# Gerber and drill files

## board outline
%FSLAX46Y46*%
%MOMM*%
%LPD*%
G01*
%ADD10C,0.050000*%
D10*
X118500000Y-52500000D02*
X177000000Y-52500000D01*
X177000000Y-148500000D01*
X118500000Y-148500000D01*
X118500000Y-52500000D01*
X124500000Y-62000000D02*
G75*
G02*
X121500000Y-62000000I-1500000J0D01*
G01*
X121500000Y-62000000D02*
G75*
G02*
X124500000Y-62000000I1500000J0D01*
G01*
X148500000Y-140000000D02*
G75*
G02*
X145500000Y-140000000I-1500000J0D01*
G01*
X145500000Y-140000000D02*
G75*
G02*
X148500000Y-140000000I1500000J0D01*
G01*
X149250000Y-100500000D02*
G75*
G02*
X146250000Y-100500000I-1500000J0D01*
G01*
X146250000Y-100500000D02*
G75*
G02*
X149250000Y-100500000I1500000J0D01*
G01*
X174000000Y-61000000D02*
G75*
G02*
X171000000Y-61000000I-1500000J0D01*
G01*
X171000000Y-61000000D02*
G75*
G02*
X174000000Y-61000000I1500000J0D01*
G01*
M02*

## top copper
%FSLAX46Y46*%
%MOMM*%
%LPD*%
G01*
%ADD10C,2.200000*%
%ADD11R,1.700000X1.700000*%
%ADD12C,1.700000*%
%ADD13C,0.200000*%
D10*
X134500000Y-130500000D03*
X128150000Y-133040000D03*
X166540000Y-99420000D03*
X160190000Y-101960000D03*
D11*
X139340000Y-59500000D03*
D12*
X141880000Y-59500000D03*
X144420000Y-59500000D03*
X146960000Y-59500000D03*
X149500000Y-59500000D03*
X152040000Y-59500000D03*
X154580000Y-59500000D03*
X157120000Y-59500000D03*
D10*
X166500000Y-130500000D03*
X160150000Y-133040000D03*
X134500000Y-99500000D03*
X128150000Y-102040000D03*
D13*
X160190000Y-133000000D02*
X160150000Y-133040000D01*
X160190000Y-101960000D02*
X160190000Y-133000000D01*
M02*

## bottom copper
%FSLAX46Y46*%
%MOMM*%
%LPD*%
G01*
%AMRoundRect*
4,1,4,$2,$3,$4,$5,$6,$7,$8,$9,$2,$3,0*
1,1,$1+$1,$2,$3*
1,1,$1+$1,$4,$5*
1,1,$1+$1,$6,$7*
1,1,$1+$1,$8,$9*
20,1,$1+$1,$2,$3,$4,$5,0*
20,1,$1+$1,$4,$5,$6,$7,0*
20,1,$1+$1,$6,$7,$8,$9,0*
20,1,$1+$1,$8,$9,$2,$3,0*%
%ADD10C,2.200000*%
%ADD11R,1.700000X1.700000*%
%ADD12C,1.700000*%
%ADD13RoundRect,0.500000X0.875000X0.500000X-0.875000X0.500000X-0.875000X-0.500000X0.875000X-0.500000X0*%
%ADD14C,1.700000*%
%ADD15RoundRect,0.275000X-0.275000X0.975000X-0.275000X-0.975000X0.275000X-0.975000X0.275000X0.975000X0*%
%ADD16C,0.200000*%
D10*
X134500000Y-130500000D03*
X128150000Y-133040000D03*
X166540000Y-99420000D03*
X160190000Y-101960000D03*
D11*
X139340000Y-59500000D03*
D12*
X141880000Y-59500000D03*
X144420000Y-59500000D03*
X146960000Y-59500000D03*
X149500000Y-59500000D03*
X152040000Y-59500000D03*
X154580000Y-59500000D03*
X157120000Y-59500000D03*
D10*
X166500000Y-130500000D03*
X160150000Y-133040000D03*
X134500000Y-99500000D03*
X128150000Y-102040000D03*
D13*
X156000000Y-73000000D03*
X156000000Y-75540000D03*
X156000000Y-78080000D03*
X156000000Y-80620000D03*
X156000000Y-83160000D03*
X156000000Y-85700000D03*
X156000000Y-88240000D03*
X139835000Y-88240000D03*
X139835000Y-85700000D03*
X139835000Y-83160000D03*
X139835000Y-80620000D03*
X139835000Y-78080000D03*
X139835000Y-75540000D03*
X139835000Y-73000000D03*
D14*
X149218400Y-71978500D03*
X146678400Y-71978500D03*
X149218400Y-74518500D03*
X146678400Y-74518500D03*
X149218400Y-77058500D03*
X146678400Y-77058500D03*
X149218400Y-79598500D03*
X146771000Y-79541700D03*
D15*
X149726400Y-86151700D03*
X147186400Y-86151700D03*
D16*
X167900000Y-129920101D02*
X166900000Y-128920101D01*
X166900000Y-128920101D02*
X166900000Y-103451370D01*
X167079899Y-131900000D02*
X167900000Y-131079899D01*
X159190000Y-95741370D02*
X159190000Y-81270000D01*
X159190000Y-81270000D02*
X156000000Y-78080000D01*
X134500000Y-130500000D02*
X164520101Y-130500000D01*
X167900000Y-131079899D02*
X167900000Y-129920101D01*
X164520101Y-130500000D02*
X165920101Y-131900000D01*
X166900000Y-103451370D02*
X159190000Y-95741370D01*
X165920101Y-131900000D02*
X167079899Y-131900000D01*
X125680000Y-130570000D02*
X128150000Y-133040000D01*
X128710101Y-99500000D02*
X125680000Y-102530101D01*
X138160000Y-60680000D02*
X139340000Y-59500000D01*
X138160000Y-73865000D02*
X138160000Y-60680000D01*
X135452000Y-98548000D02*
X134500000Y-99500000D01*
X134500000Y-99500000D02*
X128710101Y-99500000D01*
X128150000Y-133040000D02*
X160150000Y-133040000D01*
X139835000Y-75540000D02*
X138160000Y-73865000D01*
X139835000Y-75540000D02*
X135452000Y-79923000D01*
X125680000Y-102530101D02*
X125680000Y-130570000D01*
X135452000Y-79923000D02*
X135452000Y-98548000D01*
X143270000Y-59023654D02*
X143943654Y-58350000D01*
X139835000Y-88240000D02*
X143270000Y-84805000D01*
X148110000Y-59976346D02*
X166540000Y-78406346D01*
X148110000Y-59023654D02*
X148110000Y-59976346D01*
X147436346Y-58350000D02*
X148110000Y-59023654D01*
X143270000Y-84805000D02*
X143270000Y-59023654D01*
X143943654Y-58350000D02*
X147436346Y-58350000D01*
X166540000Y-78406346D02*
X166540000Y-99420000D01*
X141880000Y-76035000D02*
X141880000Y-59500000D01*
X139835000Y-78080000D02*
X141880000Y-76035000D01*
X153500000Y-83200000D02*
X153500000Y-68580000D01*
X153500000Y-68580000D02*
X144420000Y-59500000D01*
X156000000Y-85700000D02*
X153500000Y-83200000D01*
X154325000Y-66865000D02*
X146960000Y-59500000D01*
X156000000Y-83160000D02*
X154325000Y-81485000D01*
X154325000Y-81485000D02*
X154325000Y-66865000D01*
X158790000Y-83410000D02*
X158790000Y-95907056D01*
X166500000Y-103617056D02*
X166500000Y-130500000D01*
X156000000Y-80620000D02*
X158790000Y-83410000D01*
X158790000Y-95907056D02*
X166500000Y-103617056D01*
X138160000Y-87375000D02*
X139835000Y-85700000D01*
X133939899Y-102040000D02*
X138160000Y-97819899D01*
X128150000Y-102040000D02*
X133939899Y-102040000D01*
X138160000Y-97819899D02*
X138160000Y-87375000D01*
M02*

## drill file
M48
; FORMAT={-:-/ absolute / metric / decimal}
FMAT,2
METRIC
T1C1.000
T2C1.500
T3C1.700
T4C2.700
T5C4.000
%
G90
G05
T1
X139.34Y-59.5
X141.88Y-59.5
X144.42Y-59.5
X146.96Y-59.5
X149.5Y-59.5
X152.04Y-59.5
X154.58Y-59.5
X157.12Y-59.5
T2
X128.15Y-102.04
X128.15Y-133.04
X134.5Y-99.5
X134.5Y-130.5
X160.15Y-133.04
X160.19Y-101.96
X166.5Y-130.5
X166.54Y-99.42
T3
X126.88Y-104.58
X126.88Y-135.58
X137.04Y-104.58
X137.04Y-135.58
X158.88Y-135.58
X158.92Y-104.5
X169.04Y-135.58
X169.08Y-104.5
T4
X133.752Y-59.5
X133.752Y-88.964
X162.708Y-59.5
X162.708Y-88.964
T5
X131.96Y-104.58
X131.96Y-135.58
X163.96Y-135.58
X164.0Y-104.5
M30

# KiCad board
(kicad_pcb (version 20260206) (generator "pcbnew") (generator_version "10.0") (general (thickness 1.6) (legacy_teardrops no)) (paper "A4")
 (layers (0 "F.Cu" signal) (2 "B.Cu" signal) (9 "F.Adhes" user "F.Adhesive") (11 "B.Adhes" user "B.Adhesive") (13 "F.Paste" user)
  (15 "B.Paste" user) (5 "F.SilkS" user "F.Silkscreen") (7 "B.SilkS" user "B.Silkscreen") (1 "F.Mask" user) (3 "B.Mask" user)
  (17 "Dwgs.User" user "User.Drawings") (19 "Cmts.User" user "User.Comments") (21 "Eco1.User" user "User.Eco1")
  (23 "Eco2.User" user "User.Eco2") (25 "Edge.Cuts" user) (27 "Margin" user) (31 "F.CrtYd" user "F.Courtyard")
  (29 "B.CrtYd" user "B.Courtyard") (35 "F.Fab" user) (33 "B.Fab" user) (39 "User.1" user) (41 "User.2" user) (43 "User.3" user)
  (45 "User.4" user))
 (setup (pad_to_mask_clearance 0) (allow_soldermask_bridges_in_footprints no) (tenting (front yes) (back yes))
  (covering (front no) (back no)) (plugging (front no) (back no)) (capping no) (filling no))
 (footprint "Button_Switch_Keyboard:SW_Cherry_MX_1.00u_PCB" (layer "F.Cu") (at 134.5 130.5)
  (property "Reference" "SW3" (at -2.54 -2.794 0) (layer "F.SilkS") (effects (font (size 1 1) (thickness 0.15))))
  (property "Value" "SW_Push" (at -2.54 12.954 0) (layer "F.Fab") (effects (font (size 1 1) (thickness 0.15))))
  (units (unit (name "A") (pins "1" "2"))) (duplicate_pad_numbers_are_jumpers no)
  (pad "" np_thru_hole circle (at -7.62 5.08) (size 1.7 1.7) (drill 1.7) (layers "*.Cu" "*.Mask"))
  (pad "" np_thru_hole circle (at -2.54 5.08) (size 4 4) (drill 4) (layers "*.Cu" "*.Mask"))
  (pad "" np_thru_hole circle (at 2.54 5.08) (size 1.7 1.7) (drill 1.7) (layers "*.Cu" "*.Mask"))
  (pad "1" thru_hole circle (at 0 0) (size 2.2 2.2) (drill 1.5) (layers "*.Cu" "*.Mask") (remove_unused_layers no)
   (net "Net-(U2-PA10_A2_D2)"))
  (pad "2" thru_hole circle (at -6.35 2.54) (size 2.2 2.2) (drill 1.5) (layers "*.Cu" "*.Mask") (remove_unused_layers no) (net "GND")))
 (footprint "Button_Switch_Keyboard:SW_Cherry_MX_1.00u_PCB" (layer "F.Cu") (at 166.54 99.42)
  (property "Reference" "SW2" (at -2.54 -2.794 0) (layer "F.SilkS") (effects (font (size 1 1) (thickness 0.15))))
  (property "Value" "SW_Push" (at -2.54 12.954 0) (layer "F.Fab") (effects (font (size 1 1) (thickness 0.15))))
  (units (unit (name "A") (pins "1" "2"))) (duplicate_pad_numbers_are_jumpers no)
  (pad "" np_thru_hole circle (at -7.62 5.08) (size 1.7 1.7) (drill 1.7) (layers "*.Cu" "*.Mask"))
  (pad "" np_thru_hole circle (at -2.54 5.08) (size 4 4) (drill 4) (layers "*.Cu" "*.Mask"))
  (pad "" np_thru_hole circle (at 2.54 5.08) (size 1.7 1.7) (drill 1.7) (layers "*.Cu" "*.Mask"))
  (pad "1" thru_hole circle (at 0 0) (size 2.2 2.2) (drill 1.5) (layers "*.Cu" "*.Mask") (remove_unused_layers no)
   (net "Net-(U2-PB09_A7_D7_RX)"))
  (pad "2" thru_hole circle (at -6.35 2.54) (size 2.2 2.2) (drill 1.5) (layers "*.Cu" "*.Mask") (remove_unused_layers no) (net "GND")))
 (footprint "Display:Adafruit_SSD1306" (layer "F.Cu") (at 139.34 59.5)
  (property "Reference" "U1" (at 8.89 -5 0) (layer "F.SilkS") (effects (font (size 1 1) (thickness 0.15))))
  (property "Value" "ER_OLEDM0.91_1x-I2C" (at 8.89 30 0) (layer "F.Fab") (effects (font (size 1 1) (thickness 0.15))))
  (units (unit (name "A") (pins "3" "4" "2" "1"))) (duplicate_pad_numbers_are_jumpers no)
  (pad "" np_thru_hole circle (at -5.588 0) (size 2.7 2.7) (drill 2.7) (layers "*.Cu" "*.Mask"))
  (pad "" np_thru_hole circle (at -5.588 29.464) (size 2.7 2.7) (drill 2.7) (layers "*.Cu" "*.Mask"))
  (pad "" np_thru_hole circle (at 23.368 0) (size 2.7 2.7) (drill 2.7) (layers "*.Cu" "*.Mask"))
  (pad "" np_thru_hole circle (at 23.368 29.464) (size 2.7 2.7) (drill 2.7) (layers "*.Cu" "*.Mask"))
  (pad "1" thru_hole rect (at 0 0) (size 1.7 1.7) (drill 1) (layers "*.Cu" "*.Mask") (remove_unused_layers no) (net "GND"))
  (pad "2" thru_hole circle (at 2.54 0) (size 1.7 1.7) (drill 1) (layers "*.Cu" "*.Mask") (remove_unused_layers no) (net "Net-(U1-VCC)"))
  (pad "3" thru_hole circle (at 5.08 0) (size 1.7 1.7) (drill 1) (layers "*.Cu" "*.Mask") (remove_unused_layers no) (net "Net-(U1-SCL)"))
  (pad "4" thru_hole circle (at 7.62 0) (size 1.7 1.7) (drill 1) (layers "*.Cu" "*.Mask") (remove_unused_layers no) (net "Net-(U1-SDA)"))
  (pad "5" thru_hole circle (at 10.16 0) (size 1.7 1.7) (drill 1) (layers "*.Cu" "*.Mask") (remove_unused_layers no))
  (pad "6" thru_hole circle (at 12.7 0) (size 1.7 1.7) (drill 1) (layers "*.Cu" "*.Mask") (remove_unused_layers no))
  (pad "7" thru_hole circle (at 15.24 0) (size 1.7 1.7) (drill 1) (layers "*.Cu" "*.Mask") (remove_unused_layers no))
  (pad "8" thru_hole circle (at 17.78 0) (size 1.7 1.7) (drill 1) (layers "*.Cu" "*.Mask") (remove_unused_layers no)))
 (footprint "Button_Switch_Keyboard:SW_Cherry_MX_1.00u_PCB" (layer "F.Cu") (at 166.5 130.5)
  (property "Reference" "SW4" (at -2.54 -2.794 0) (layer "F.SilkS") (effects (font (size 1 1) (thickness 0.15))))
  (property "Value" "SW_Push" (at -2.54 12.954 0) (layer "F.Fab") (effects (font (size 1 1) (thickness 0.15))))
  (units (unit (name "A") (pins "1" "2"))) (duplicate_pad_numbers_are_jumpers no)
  (pad "" np_thru_hole circle (at -7.62 5.08) (size 1.7 1.7) (drill 1.7) (layers "*.Cu" "*.Mask"))
  (pad "" np_thru_hole circle (at -2.54 5.08) (size 4 4) (drill 4) (layers "*.Cu" "*.Mask"))
  (pad "" np_thru_hole circle (at 2.54 5.08) (size 1.7 1.7) (drill 1.7) (layers "*.Cu" "*.Mask"))
  (pad "1" thru_hole circle (at 0 0) (size 2.2 2.2) (drill 1.5) (layers "*.Cu" "*.Mask") (remove_unused_layers no)
   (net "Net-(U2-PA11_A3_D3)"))
  (pad "2" thru_hole circle (at -6.35 2.54) (size 2.2 2.2) (drill 1.5) (layers "*.Cu" "*.Mask") (remove_unused_layers no) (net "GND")))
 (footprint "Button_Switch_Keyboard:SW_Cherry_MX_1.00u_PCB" (layer "F.Cu") (at 134.5 99.5)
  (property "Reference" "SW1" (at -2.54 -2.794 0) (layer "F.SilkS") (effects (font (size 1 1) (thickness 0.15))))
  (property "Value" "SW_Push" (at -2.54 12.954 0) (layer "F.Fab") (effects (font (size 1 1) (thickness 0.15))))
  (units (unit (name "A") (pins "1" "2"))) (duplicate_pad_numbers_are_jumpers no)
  (pad "" np_thru_hole circle (at -7.62 5.08) (size 1.7 1.7) (drill 1.7) (layers "*.Cu" "*.Mask"))
  (pad "" np_thru_hole circle (at -2.54 5.08) (size 4 4) (drill 4) (layers "*.Cu" "*.Mask"))
  (pad "" np_thru_hole circle (at 2.54 5.08) (size 1.7 1.7) (drill 1.7) (layers "*.Cu" "*.Mask"))
  (pad "1" thru_hole circle (at 0 0) (size 2.2 2.2) (drill 1.5) (layers "*.Cu" "*.Mask") (remove_unused_layers no) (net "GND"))
  (pad "2" thru_hole circle (at -6.35 2.54) (size 2.2 2.2) (drill 1.5) (layers "*.Cu" "*.Mask") (remove_unused_layers no)
   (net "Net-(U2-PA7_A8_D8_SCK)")))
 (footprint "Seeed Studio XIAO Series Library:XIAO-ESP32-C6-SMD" (layer "B.Cu") (at 156.835 91.12 180)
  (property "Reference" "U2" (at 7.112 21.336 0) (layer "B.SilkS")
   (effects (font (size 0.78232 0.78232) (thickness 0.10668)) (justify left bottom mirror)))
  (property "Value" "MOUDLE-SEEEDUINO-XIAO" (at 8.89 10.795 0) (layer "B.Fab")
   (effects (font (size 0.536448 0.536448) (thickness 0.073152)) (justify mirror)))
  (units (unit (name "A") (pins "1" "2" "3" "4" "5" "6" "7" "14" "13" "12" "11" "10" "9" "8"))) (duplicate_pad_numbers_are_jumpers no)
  (pad "1" smd roundrect (at 0.835 18.12 180) (size 2.75 2) (layers "B.Cu" "B.Mask" "B.Paste") (roundrect_rratio 0.25)
   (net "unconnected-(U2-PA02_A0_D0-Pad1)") (solder_mask_margin 0.0508) (thermal_bridge_angle 45))
  (pad "2" smd roundrect (at 0.835 15.58 180) (size 2.75 2) (layers "B.Cu" "B.Mask" "B.Paste") (roundrect_rratio 0.25)
   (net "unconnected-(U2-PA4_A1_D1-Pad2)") (solder_mask_margin 0.0508) (thermal_bridge_angle 45))
  (pad "3" smd roundrect (at 0.835 13.04 180) (size 2.75 2) (layers "B.Cu" "B.Mask" "B.Paste") (roundrect_rratio 0.25)
   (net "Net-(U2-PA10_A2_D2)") (solder_mask_margin 0.0508) (thermal_bridge_angle 45))
  (pad "4" smd roundrect (at 0.835 10.5 180) (size 2.75 2) (layers "B.Cu" "B.Mask" "B.Paste") (roundrect_rratio 0.25)
   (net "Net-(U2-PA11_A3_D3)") (solder_mask_margin 0.0508) (thermal_bridge_angle 45))
  (pad "5" smd roundrect (at 0.835 7.96 180) (size 2.75 2) (layers "B.Cu" "B.Mask" "B.Paste") (roundrect_rratio 0.25) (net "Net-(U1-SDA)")
   (solder_mask_margin 0.0508) (thermal_bridge_angle 45))
  (pad "6" smd roundrect (at 0.835 5.42 180) (size 2.75 2) (layers "B.Cu" "B.Mask" "B.Paste") (roundrect_rratio 0.25) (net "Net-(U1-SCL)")
   (solder_mask_margin 0.0508) (thermal_bridge_angle 45))
  (pad "7" smd roundrect (at 0.835 2.88 180) (size 2.75 2) (layers "B.Cu" "B.Mask" "B.Paste") (roundrect_rratio 0.25)
   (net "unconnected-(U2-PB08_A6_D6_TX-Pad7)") (solder_mask_margin 0.0508) (thermal_bridge_angle 45))
  (pad "8" smd roundrect (at 17 2.88 180) (size 2.75 2) (layers "B.Cu" "B.Mask" "B.Paste") (roundrect_rratio 0.25)
   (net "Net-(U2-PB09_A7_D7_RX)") (solder_mask_margin 0.0508) (thermal_bridge_angle 45))
  (pad "9" smd roundrect (at 17 5.42 180) (size 2.75 2) (layers "B.Cu" "B.Mask" "B.Paste") (roundrect_rratio 0.25)
   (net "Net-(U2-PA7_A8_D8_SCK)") (solder_mask_margin 0.0508) (thermal_bridge_angle 45))
  (pad "10" smd roundrect (at 17 7.96 180) (size 2.75 2) (layers "B.Cu" "B.Mask" "B.Paste") (roundrect_rratio 0.25)
   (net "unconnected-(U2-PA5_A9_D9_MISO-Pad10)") (solder_mask_margin 0.0508) (thermal_bridge_angle 45))
  (pad "11" smd roundrect (at 17 10.5 180) (size 2.75 2) (layers "B.Cu" "B.Mask" "B.Paste") (roundrect_rratio 0.25)
   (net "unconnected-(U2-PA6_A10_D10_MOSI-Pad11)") (solder_mask_margin 0.0508) (thermal_bridge_angle 45))
  (pad "12" smd roundrect (at 17 13.04 180) (size 2.75 2) (layers "B.Cu" "B.Mask" "B.Paste") (roundrect_rratio 0.25) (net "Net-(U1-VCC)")
   (solder_mask_margin 0.0508) (thermal_bridge_angle 45))
  (pad "13" smd roundrect (at 17 15.58 180) (size 2.75 2) (layers "B.Cu" "B.Mask" "B.Paste") (roundrect_rratio 0.25) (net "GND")
   (solder_mask_margin 0.0508) (thermal_bridge_angle 45))
  (pad "14" smd roundrect (at 17 18.12 180) (size 2.75 2) (layers "B.Cu" "B.Mask" "B.Paste") (roundrect_rratio 0.25)
   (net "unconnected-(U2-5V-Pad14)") (solder_mask_margin 0.0508) (thermal_bridge_angle 45))
  (pad "15" smd circle (at 7.6166 19.1415 180) (size 1.7 1.7) (layers "B.Cu" "B.Mask" "B.Paste"))
  (pad "16" smd circle (at 10.1566 19.1415 180) (size 1.7 1.7) (layers "B.Cu" "B.Mask" "B.Paste"))
  (pad "17" smd circle (at 7.6166 16.6015 180) (size 1.7 1.7) (layers "B.Cu" "B.Mask" "B.Paste"))
  (pad "18" smd circle (at 10.1566 16.6015 180) (size 1.7 1.7) (layers "B.Cu" "B.Mask" "B.Paste"))
  (pad "19" smd circle (at 7.6166 14.0615 180) (size 1.7 1.7) (layers "B.Cu" "B.Mask" "B.Paste"))
  (pad "20" smd circle (at 10.1566 14.0615 180) (size 1.7 1.7) (layers "B.Cu" "B.Mask" "B.Paste"))
  (pad "21" smd circle (at 7.6166 11.5215 180) (size 1.7 1.7) (layers "B.Cu" "B.Mask" "B.Paste"))
  (pad "22" smd circle (at 10.064 11.5783 180) (size 1.7 1.7) (layers "B.Cu" "B.Mask" "B.Paste"))
  (pad "23" smd roundrect (at 7.1086 4.9683 270) (size 2.5 1.1) (layers "B.Cu" "B.Mask" "B.Paste") (roundrect_rratio 0.25)
   (thermal_bridge_angle 45))
  (pad "24" smd roundrect (at 9.6486 4.9683 270) (size 2.5 1.1) (layers "B.Cu" "B.Mask" "B.Paste") (roundrect_rratio 0.25)
   (thermal_bridge_angle 45)))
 (gr_rect (start 118.5 52.5) (end 177 148.5) (stroke (width 0.05) (type default)) (fill no) (layer "Edge.Cuts"))
 (gr_circle (center 123 62) (end 123 60.5) (stroke (width 0.05) (type default)) (fill no) (layer "Edge.Cuts"))
 (gr_circle (center 147 140) (end 145.5 140) (stroke (width 0.05) (type default)) (fill no) (layer "Edge.Cuts"))
 (gr_circle (center 147.75 100.5) (end 147.75 99) (stroke (width 0.05) (type default)) (fill no) (layer "Edge.Cuts"))
 (gr_circle (center 172.5 61) (end 172.5 59.5) (stroke (width 0.05) (type default)) (fill no) (layer "Edge.Cuts"))
 (segment (start 167.9 129.920101) (end 166.9 128.920101) (width 0.2) (layer "B.Cu") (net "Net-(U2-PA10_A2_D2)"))
 (segment (start 166.9 128.920101) (end 166.9 103.45137) (width 0.2) (layer "B.Cu") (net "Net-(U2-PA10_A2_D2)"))
 (segment (start 167.079899 131.9) (end 167.9 131.079899) (width 0.2) (layer "B.Cu") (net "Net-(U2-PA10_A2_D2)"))
 (segment (start 159.19 95.74137) (end 159.19 81.27) (width 0.2) (layer "B.Cu") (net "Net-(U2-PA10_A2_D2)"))
 (segment (start 159.19 81.27) (end 156 78.08) (width 0.2) (layer "B.Cu") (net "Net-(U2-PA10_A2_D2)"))
 (segment (start 134.5 130.5) (end 164.520101 130.5) (width 0.2) (layer "B.Cu") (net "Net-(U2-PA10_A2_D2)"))
 (segment (start 167.9 131.079899) (end 167.9 129.920101) (width 0.2) (layer "B.Cu") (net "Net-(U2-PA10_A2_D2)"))
 (segment (start 164.520101 130.5) (end 165.920101 131.9) (width 0.2) (layer "B.Cu") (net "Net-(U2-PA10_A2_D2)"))
 (segment (start 166.9 103.45137) (end 159.19 95.74137) (width 0.2) (layer "B.Cu") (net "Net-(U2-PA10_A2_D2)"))
 (segment (start 165.920101 131.9) (end 167.079899 131.9) (width 0.2) (layer "B.Cu") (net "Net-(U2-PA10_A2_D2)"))
 (segment (start 160.19 133) (end 160.15 133.04) (width 0.2) (layer "F.Cu") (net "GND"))
 (segment (start 160.19 101.96) (end 160.19 133) (width 0.2) (layer "F.Cu") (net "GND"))
 (segment (start 125.68 130.57) (end 128.15 133.04) (width 0.2) (layer "B.Cu") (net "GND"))
 (segment (start 128.710101 99.5) (end 125.68 102.530101) (width 0.2) (layer "B.Cu") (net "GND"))
 (segment (start 138.16 60.68) (end 139.34 59.5) (width 0.2) (layer "B.Cu") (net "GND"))
 (segment (start 138.16 73.865) (end 138.16 60.68) (width 0.2) (layer "B.Cu") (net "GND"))
 (segment (start 135.452 98.548) (end 134.5 99.5) (width 0.2) (layer "B.Cu") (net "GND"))
 (segment (start 134.5 99.5) (end 128.710101 99.5) (width 0.2) (layer "B.Cu") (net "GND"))
 (segment (start 128.15 133.04) (end 160.15 133.04) (width 0.2) (layer "B.Cu") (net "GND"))
 (segment (start 139.835 75.54) (end 138.16 73.865) (width 0.2) (layer "B.Cu") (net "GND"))
 (segment (start 139.835 75.54) (end 135.452 79.923) (width 0.2) (layer "B.Cu") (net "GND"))
 (segment (start 125.68 102.530101) (end 125.68 130.57) (width 0.2) (layer "B.Cu") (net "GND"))
 (segment (start 135.452 79.923) (end 135.452 98.548) (width 0.2) (layer "B.Cu") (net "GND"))
 (segment (start 143.27 59.023654) (end 143.943654 58.35) (width 0.2) (layer "B.Cu") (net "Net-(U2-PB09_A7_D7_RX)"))
 (segment (start 139.835 88.24) (end 143.27 84.805) (width 0.2) (layer "B.Cu") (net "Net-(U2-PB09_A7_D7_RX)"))
 (segment (start 148.11 59.976346) (end 166.54 78.406346) (width 0.2) (layer "B.Cu") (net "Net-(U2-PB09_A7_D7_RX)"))
 (segment (start 148.11 59.023654) (end 148.11 59.976346) (width 0.2) (layer "B.Cu") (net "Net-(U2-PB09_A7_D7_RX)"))
 (segment (start 147.436346 58.35) (end 148.11 59.023654) (width 0.2) (layer "B.Cu") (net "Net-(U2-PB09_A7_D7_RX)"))
 (segment (start 143.27 84.805) (end 143.27 59.023654) (width 0.2) (layer "B.Cu") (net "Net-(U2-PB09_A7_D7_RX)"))
 (segment (start 143.943654 58.35) (end 147.436346 58.35) (width 0.2) (layer "B.Cu") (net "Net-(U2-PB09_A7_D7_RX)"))
 (segment (start 166.54 78.406346) (end 166.54 99.42) (width 0.2) (layer "B.Cu") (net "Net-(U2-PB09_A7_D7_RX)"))
 (segment (start 141.88 76.035) (end 141.88 59.5) (width 0.2) (layer "B.Cu") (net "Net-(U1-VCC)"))
 (segment (start 139.835 78.08) (end 141.88 76.035) (width 0.2) (layer "B.Cu") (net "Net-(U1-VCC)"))
 (segment (start 153.5 83.2) (end 153.5 68.58) (width 0.2) (layer "B.Cu") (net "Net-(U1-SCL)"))
 (segment (start 153.5 68.58) (end 144.42 59.5) (width 0.2) (layer "B.Cu") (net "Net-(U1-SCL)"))
 (segment (start 156 85.7) (end 153.5 83.2) (width 0.2) (layer "B.Cu") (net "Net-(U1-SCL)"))
 (segment (start 154.325 66.865) (end 146.96 59.5) (width 0.2) (layer "B.Cu") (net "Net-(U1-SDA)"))
 (segment (start 156 83.16) (end 154.325 81.485) (width 0.2) (layer "B.Cu") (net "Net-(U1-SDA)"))
 (segment (start 154.325 81.485) (end 154.325 66.865) (width 0.2) (layer "B.Cu") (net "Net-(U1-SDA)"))
 (segment (start 158.79 83.41) (end 158.79 95.907056) (width 0.2) (layer "B.Cu") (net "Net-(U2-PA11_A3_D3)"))
 (segment (start 166.5 103.617056) (end 166.5 130.5) (width 0.2) (layer "B.Cu") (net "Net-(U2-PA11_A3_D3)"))
 (segment (start 156 80.62) (end 158.79 83.41) (width 0.2) (layer "B.Cu") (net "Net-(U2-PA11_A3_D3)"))
 (segment (start 158.79 95.907056) (end 166.5 103.617056) (width 0.2) (layer "B.Cu") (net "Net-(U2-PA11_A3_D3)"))
 (segment (start 138.16 87.375) (end 139.835 85.7) (width 0.2) (layer "B.Cu") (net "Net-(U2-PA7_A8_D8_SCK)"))
 (segment (start 133.939899 102.04) (end 138.16 97.819899) (width 0.2) (layer "B.Cu") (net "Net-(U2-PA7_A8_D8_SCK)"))
 (segment (start 128.15 102.04) (end 133.939899 102.04) (width 0.2) (layer "B.Cu") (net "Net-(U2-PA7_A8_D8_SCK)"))
 (segment (start 138.16 97.819899) (end 138.16 87.375) (width 0.2) (layer "B.Cu") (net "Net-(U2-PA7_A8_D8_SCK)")))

